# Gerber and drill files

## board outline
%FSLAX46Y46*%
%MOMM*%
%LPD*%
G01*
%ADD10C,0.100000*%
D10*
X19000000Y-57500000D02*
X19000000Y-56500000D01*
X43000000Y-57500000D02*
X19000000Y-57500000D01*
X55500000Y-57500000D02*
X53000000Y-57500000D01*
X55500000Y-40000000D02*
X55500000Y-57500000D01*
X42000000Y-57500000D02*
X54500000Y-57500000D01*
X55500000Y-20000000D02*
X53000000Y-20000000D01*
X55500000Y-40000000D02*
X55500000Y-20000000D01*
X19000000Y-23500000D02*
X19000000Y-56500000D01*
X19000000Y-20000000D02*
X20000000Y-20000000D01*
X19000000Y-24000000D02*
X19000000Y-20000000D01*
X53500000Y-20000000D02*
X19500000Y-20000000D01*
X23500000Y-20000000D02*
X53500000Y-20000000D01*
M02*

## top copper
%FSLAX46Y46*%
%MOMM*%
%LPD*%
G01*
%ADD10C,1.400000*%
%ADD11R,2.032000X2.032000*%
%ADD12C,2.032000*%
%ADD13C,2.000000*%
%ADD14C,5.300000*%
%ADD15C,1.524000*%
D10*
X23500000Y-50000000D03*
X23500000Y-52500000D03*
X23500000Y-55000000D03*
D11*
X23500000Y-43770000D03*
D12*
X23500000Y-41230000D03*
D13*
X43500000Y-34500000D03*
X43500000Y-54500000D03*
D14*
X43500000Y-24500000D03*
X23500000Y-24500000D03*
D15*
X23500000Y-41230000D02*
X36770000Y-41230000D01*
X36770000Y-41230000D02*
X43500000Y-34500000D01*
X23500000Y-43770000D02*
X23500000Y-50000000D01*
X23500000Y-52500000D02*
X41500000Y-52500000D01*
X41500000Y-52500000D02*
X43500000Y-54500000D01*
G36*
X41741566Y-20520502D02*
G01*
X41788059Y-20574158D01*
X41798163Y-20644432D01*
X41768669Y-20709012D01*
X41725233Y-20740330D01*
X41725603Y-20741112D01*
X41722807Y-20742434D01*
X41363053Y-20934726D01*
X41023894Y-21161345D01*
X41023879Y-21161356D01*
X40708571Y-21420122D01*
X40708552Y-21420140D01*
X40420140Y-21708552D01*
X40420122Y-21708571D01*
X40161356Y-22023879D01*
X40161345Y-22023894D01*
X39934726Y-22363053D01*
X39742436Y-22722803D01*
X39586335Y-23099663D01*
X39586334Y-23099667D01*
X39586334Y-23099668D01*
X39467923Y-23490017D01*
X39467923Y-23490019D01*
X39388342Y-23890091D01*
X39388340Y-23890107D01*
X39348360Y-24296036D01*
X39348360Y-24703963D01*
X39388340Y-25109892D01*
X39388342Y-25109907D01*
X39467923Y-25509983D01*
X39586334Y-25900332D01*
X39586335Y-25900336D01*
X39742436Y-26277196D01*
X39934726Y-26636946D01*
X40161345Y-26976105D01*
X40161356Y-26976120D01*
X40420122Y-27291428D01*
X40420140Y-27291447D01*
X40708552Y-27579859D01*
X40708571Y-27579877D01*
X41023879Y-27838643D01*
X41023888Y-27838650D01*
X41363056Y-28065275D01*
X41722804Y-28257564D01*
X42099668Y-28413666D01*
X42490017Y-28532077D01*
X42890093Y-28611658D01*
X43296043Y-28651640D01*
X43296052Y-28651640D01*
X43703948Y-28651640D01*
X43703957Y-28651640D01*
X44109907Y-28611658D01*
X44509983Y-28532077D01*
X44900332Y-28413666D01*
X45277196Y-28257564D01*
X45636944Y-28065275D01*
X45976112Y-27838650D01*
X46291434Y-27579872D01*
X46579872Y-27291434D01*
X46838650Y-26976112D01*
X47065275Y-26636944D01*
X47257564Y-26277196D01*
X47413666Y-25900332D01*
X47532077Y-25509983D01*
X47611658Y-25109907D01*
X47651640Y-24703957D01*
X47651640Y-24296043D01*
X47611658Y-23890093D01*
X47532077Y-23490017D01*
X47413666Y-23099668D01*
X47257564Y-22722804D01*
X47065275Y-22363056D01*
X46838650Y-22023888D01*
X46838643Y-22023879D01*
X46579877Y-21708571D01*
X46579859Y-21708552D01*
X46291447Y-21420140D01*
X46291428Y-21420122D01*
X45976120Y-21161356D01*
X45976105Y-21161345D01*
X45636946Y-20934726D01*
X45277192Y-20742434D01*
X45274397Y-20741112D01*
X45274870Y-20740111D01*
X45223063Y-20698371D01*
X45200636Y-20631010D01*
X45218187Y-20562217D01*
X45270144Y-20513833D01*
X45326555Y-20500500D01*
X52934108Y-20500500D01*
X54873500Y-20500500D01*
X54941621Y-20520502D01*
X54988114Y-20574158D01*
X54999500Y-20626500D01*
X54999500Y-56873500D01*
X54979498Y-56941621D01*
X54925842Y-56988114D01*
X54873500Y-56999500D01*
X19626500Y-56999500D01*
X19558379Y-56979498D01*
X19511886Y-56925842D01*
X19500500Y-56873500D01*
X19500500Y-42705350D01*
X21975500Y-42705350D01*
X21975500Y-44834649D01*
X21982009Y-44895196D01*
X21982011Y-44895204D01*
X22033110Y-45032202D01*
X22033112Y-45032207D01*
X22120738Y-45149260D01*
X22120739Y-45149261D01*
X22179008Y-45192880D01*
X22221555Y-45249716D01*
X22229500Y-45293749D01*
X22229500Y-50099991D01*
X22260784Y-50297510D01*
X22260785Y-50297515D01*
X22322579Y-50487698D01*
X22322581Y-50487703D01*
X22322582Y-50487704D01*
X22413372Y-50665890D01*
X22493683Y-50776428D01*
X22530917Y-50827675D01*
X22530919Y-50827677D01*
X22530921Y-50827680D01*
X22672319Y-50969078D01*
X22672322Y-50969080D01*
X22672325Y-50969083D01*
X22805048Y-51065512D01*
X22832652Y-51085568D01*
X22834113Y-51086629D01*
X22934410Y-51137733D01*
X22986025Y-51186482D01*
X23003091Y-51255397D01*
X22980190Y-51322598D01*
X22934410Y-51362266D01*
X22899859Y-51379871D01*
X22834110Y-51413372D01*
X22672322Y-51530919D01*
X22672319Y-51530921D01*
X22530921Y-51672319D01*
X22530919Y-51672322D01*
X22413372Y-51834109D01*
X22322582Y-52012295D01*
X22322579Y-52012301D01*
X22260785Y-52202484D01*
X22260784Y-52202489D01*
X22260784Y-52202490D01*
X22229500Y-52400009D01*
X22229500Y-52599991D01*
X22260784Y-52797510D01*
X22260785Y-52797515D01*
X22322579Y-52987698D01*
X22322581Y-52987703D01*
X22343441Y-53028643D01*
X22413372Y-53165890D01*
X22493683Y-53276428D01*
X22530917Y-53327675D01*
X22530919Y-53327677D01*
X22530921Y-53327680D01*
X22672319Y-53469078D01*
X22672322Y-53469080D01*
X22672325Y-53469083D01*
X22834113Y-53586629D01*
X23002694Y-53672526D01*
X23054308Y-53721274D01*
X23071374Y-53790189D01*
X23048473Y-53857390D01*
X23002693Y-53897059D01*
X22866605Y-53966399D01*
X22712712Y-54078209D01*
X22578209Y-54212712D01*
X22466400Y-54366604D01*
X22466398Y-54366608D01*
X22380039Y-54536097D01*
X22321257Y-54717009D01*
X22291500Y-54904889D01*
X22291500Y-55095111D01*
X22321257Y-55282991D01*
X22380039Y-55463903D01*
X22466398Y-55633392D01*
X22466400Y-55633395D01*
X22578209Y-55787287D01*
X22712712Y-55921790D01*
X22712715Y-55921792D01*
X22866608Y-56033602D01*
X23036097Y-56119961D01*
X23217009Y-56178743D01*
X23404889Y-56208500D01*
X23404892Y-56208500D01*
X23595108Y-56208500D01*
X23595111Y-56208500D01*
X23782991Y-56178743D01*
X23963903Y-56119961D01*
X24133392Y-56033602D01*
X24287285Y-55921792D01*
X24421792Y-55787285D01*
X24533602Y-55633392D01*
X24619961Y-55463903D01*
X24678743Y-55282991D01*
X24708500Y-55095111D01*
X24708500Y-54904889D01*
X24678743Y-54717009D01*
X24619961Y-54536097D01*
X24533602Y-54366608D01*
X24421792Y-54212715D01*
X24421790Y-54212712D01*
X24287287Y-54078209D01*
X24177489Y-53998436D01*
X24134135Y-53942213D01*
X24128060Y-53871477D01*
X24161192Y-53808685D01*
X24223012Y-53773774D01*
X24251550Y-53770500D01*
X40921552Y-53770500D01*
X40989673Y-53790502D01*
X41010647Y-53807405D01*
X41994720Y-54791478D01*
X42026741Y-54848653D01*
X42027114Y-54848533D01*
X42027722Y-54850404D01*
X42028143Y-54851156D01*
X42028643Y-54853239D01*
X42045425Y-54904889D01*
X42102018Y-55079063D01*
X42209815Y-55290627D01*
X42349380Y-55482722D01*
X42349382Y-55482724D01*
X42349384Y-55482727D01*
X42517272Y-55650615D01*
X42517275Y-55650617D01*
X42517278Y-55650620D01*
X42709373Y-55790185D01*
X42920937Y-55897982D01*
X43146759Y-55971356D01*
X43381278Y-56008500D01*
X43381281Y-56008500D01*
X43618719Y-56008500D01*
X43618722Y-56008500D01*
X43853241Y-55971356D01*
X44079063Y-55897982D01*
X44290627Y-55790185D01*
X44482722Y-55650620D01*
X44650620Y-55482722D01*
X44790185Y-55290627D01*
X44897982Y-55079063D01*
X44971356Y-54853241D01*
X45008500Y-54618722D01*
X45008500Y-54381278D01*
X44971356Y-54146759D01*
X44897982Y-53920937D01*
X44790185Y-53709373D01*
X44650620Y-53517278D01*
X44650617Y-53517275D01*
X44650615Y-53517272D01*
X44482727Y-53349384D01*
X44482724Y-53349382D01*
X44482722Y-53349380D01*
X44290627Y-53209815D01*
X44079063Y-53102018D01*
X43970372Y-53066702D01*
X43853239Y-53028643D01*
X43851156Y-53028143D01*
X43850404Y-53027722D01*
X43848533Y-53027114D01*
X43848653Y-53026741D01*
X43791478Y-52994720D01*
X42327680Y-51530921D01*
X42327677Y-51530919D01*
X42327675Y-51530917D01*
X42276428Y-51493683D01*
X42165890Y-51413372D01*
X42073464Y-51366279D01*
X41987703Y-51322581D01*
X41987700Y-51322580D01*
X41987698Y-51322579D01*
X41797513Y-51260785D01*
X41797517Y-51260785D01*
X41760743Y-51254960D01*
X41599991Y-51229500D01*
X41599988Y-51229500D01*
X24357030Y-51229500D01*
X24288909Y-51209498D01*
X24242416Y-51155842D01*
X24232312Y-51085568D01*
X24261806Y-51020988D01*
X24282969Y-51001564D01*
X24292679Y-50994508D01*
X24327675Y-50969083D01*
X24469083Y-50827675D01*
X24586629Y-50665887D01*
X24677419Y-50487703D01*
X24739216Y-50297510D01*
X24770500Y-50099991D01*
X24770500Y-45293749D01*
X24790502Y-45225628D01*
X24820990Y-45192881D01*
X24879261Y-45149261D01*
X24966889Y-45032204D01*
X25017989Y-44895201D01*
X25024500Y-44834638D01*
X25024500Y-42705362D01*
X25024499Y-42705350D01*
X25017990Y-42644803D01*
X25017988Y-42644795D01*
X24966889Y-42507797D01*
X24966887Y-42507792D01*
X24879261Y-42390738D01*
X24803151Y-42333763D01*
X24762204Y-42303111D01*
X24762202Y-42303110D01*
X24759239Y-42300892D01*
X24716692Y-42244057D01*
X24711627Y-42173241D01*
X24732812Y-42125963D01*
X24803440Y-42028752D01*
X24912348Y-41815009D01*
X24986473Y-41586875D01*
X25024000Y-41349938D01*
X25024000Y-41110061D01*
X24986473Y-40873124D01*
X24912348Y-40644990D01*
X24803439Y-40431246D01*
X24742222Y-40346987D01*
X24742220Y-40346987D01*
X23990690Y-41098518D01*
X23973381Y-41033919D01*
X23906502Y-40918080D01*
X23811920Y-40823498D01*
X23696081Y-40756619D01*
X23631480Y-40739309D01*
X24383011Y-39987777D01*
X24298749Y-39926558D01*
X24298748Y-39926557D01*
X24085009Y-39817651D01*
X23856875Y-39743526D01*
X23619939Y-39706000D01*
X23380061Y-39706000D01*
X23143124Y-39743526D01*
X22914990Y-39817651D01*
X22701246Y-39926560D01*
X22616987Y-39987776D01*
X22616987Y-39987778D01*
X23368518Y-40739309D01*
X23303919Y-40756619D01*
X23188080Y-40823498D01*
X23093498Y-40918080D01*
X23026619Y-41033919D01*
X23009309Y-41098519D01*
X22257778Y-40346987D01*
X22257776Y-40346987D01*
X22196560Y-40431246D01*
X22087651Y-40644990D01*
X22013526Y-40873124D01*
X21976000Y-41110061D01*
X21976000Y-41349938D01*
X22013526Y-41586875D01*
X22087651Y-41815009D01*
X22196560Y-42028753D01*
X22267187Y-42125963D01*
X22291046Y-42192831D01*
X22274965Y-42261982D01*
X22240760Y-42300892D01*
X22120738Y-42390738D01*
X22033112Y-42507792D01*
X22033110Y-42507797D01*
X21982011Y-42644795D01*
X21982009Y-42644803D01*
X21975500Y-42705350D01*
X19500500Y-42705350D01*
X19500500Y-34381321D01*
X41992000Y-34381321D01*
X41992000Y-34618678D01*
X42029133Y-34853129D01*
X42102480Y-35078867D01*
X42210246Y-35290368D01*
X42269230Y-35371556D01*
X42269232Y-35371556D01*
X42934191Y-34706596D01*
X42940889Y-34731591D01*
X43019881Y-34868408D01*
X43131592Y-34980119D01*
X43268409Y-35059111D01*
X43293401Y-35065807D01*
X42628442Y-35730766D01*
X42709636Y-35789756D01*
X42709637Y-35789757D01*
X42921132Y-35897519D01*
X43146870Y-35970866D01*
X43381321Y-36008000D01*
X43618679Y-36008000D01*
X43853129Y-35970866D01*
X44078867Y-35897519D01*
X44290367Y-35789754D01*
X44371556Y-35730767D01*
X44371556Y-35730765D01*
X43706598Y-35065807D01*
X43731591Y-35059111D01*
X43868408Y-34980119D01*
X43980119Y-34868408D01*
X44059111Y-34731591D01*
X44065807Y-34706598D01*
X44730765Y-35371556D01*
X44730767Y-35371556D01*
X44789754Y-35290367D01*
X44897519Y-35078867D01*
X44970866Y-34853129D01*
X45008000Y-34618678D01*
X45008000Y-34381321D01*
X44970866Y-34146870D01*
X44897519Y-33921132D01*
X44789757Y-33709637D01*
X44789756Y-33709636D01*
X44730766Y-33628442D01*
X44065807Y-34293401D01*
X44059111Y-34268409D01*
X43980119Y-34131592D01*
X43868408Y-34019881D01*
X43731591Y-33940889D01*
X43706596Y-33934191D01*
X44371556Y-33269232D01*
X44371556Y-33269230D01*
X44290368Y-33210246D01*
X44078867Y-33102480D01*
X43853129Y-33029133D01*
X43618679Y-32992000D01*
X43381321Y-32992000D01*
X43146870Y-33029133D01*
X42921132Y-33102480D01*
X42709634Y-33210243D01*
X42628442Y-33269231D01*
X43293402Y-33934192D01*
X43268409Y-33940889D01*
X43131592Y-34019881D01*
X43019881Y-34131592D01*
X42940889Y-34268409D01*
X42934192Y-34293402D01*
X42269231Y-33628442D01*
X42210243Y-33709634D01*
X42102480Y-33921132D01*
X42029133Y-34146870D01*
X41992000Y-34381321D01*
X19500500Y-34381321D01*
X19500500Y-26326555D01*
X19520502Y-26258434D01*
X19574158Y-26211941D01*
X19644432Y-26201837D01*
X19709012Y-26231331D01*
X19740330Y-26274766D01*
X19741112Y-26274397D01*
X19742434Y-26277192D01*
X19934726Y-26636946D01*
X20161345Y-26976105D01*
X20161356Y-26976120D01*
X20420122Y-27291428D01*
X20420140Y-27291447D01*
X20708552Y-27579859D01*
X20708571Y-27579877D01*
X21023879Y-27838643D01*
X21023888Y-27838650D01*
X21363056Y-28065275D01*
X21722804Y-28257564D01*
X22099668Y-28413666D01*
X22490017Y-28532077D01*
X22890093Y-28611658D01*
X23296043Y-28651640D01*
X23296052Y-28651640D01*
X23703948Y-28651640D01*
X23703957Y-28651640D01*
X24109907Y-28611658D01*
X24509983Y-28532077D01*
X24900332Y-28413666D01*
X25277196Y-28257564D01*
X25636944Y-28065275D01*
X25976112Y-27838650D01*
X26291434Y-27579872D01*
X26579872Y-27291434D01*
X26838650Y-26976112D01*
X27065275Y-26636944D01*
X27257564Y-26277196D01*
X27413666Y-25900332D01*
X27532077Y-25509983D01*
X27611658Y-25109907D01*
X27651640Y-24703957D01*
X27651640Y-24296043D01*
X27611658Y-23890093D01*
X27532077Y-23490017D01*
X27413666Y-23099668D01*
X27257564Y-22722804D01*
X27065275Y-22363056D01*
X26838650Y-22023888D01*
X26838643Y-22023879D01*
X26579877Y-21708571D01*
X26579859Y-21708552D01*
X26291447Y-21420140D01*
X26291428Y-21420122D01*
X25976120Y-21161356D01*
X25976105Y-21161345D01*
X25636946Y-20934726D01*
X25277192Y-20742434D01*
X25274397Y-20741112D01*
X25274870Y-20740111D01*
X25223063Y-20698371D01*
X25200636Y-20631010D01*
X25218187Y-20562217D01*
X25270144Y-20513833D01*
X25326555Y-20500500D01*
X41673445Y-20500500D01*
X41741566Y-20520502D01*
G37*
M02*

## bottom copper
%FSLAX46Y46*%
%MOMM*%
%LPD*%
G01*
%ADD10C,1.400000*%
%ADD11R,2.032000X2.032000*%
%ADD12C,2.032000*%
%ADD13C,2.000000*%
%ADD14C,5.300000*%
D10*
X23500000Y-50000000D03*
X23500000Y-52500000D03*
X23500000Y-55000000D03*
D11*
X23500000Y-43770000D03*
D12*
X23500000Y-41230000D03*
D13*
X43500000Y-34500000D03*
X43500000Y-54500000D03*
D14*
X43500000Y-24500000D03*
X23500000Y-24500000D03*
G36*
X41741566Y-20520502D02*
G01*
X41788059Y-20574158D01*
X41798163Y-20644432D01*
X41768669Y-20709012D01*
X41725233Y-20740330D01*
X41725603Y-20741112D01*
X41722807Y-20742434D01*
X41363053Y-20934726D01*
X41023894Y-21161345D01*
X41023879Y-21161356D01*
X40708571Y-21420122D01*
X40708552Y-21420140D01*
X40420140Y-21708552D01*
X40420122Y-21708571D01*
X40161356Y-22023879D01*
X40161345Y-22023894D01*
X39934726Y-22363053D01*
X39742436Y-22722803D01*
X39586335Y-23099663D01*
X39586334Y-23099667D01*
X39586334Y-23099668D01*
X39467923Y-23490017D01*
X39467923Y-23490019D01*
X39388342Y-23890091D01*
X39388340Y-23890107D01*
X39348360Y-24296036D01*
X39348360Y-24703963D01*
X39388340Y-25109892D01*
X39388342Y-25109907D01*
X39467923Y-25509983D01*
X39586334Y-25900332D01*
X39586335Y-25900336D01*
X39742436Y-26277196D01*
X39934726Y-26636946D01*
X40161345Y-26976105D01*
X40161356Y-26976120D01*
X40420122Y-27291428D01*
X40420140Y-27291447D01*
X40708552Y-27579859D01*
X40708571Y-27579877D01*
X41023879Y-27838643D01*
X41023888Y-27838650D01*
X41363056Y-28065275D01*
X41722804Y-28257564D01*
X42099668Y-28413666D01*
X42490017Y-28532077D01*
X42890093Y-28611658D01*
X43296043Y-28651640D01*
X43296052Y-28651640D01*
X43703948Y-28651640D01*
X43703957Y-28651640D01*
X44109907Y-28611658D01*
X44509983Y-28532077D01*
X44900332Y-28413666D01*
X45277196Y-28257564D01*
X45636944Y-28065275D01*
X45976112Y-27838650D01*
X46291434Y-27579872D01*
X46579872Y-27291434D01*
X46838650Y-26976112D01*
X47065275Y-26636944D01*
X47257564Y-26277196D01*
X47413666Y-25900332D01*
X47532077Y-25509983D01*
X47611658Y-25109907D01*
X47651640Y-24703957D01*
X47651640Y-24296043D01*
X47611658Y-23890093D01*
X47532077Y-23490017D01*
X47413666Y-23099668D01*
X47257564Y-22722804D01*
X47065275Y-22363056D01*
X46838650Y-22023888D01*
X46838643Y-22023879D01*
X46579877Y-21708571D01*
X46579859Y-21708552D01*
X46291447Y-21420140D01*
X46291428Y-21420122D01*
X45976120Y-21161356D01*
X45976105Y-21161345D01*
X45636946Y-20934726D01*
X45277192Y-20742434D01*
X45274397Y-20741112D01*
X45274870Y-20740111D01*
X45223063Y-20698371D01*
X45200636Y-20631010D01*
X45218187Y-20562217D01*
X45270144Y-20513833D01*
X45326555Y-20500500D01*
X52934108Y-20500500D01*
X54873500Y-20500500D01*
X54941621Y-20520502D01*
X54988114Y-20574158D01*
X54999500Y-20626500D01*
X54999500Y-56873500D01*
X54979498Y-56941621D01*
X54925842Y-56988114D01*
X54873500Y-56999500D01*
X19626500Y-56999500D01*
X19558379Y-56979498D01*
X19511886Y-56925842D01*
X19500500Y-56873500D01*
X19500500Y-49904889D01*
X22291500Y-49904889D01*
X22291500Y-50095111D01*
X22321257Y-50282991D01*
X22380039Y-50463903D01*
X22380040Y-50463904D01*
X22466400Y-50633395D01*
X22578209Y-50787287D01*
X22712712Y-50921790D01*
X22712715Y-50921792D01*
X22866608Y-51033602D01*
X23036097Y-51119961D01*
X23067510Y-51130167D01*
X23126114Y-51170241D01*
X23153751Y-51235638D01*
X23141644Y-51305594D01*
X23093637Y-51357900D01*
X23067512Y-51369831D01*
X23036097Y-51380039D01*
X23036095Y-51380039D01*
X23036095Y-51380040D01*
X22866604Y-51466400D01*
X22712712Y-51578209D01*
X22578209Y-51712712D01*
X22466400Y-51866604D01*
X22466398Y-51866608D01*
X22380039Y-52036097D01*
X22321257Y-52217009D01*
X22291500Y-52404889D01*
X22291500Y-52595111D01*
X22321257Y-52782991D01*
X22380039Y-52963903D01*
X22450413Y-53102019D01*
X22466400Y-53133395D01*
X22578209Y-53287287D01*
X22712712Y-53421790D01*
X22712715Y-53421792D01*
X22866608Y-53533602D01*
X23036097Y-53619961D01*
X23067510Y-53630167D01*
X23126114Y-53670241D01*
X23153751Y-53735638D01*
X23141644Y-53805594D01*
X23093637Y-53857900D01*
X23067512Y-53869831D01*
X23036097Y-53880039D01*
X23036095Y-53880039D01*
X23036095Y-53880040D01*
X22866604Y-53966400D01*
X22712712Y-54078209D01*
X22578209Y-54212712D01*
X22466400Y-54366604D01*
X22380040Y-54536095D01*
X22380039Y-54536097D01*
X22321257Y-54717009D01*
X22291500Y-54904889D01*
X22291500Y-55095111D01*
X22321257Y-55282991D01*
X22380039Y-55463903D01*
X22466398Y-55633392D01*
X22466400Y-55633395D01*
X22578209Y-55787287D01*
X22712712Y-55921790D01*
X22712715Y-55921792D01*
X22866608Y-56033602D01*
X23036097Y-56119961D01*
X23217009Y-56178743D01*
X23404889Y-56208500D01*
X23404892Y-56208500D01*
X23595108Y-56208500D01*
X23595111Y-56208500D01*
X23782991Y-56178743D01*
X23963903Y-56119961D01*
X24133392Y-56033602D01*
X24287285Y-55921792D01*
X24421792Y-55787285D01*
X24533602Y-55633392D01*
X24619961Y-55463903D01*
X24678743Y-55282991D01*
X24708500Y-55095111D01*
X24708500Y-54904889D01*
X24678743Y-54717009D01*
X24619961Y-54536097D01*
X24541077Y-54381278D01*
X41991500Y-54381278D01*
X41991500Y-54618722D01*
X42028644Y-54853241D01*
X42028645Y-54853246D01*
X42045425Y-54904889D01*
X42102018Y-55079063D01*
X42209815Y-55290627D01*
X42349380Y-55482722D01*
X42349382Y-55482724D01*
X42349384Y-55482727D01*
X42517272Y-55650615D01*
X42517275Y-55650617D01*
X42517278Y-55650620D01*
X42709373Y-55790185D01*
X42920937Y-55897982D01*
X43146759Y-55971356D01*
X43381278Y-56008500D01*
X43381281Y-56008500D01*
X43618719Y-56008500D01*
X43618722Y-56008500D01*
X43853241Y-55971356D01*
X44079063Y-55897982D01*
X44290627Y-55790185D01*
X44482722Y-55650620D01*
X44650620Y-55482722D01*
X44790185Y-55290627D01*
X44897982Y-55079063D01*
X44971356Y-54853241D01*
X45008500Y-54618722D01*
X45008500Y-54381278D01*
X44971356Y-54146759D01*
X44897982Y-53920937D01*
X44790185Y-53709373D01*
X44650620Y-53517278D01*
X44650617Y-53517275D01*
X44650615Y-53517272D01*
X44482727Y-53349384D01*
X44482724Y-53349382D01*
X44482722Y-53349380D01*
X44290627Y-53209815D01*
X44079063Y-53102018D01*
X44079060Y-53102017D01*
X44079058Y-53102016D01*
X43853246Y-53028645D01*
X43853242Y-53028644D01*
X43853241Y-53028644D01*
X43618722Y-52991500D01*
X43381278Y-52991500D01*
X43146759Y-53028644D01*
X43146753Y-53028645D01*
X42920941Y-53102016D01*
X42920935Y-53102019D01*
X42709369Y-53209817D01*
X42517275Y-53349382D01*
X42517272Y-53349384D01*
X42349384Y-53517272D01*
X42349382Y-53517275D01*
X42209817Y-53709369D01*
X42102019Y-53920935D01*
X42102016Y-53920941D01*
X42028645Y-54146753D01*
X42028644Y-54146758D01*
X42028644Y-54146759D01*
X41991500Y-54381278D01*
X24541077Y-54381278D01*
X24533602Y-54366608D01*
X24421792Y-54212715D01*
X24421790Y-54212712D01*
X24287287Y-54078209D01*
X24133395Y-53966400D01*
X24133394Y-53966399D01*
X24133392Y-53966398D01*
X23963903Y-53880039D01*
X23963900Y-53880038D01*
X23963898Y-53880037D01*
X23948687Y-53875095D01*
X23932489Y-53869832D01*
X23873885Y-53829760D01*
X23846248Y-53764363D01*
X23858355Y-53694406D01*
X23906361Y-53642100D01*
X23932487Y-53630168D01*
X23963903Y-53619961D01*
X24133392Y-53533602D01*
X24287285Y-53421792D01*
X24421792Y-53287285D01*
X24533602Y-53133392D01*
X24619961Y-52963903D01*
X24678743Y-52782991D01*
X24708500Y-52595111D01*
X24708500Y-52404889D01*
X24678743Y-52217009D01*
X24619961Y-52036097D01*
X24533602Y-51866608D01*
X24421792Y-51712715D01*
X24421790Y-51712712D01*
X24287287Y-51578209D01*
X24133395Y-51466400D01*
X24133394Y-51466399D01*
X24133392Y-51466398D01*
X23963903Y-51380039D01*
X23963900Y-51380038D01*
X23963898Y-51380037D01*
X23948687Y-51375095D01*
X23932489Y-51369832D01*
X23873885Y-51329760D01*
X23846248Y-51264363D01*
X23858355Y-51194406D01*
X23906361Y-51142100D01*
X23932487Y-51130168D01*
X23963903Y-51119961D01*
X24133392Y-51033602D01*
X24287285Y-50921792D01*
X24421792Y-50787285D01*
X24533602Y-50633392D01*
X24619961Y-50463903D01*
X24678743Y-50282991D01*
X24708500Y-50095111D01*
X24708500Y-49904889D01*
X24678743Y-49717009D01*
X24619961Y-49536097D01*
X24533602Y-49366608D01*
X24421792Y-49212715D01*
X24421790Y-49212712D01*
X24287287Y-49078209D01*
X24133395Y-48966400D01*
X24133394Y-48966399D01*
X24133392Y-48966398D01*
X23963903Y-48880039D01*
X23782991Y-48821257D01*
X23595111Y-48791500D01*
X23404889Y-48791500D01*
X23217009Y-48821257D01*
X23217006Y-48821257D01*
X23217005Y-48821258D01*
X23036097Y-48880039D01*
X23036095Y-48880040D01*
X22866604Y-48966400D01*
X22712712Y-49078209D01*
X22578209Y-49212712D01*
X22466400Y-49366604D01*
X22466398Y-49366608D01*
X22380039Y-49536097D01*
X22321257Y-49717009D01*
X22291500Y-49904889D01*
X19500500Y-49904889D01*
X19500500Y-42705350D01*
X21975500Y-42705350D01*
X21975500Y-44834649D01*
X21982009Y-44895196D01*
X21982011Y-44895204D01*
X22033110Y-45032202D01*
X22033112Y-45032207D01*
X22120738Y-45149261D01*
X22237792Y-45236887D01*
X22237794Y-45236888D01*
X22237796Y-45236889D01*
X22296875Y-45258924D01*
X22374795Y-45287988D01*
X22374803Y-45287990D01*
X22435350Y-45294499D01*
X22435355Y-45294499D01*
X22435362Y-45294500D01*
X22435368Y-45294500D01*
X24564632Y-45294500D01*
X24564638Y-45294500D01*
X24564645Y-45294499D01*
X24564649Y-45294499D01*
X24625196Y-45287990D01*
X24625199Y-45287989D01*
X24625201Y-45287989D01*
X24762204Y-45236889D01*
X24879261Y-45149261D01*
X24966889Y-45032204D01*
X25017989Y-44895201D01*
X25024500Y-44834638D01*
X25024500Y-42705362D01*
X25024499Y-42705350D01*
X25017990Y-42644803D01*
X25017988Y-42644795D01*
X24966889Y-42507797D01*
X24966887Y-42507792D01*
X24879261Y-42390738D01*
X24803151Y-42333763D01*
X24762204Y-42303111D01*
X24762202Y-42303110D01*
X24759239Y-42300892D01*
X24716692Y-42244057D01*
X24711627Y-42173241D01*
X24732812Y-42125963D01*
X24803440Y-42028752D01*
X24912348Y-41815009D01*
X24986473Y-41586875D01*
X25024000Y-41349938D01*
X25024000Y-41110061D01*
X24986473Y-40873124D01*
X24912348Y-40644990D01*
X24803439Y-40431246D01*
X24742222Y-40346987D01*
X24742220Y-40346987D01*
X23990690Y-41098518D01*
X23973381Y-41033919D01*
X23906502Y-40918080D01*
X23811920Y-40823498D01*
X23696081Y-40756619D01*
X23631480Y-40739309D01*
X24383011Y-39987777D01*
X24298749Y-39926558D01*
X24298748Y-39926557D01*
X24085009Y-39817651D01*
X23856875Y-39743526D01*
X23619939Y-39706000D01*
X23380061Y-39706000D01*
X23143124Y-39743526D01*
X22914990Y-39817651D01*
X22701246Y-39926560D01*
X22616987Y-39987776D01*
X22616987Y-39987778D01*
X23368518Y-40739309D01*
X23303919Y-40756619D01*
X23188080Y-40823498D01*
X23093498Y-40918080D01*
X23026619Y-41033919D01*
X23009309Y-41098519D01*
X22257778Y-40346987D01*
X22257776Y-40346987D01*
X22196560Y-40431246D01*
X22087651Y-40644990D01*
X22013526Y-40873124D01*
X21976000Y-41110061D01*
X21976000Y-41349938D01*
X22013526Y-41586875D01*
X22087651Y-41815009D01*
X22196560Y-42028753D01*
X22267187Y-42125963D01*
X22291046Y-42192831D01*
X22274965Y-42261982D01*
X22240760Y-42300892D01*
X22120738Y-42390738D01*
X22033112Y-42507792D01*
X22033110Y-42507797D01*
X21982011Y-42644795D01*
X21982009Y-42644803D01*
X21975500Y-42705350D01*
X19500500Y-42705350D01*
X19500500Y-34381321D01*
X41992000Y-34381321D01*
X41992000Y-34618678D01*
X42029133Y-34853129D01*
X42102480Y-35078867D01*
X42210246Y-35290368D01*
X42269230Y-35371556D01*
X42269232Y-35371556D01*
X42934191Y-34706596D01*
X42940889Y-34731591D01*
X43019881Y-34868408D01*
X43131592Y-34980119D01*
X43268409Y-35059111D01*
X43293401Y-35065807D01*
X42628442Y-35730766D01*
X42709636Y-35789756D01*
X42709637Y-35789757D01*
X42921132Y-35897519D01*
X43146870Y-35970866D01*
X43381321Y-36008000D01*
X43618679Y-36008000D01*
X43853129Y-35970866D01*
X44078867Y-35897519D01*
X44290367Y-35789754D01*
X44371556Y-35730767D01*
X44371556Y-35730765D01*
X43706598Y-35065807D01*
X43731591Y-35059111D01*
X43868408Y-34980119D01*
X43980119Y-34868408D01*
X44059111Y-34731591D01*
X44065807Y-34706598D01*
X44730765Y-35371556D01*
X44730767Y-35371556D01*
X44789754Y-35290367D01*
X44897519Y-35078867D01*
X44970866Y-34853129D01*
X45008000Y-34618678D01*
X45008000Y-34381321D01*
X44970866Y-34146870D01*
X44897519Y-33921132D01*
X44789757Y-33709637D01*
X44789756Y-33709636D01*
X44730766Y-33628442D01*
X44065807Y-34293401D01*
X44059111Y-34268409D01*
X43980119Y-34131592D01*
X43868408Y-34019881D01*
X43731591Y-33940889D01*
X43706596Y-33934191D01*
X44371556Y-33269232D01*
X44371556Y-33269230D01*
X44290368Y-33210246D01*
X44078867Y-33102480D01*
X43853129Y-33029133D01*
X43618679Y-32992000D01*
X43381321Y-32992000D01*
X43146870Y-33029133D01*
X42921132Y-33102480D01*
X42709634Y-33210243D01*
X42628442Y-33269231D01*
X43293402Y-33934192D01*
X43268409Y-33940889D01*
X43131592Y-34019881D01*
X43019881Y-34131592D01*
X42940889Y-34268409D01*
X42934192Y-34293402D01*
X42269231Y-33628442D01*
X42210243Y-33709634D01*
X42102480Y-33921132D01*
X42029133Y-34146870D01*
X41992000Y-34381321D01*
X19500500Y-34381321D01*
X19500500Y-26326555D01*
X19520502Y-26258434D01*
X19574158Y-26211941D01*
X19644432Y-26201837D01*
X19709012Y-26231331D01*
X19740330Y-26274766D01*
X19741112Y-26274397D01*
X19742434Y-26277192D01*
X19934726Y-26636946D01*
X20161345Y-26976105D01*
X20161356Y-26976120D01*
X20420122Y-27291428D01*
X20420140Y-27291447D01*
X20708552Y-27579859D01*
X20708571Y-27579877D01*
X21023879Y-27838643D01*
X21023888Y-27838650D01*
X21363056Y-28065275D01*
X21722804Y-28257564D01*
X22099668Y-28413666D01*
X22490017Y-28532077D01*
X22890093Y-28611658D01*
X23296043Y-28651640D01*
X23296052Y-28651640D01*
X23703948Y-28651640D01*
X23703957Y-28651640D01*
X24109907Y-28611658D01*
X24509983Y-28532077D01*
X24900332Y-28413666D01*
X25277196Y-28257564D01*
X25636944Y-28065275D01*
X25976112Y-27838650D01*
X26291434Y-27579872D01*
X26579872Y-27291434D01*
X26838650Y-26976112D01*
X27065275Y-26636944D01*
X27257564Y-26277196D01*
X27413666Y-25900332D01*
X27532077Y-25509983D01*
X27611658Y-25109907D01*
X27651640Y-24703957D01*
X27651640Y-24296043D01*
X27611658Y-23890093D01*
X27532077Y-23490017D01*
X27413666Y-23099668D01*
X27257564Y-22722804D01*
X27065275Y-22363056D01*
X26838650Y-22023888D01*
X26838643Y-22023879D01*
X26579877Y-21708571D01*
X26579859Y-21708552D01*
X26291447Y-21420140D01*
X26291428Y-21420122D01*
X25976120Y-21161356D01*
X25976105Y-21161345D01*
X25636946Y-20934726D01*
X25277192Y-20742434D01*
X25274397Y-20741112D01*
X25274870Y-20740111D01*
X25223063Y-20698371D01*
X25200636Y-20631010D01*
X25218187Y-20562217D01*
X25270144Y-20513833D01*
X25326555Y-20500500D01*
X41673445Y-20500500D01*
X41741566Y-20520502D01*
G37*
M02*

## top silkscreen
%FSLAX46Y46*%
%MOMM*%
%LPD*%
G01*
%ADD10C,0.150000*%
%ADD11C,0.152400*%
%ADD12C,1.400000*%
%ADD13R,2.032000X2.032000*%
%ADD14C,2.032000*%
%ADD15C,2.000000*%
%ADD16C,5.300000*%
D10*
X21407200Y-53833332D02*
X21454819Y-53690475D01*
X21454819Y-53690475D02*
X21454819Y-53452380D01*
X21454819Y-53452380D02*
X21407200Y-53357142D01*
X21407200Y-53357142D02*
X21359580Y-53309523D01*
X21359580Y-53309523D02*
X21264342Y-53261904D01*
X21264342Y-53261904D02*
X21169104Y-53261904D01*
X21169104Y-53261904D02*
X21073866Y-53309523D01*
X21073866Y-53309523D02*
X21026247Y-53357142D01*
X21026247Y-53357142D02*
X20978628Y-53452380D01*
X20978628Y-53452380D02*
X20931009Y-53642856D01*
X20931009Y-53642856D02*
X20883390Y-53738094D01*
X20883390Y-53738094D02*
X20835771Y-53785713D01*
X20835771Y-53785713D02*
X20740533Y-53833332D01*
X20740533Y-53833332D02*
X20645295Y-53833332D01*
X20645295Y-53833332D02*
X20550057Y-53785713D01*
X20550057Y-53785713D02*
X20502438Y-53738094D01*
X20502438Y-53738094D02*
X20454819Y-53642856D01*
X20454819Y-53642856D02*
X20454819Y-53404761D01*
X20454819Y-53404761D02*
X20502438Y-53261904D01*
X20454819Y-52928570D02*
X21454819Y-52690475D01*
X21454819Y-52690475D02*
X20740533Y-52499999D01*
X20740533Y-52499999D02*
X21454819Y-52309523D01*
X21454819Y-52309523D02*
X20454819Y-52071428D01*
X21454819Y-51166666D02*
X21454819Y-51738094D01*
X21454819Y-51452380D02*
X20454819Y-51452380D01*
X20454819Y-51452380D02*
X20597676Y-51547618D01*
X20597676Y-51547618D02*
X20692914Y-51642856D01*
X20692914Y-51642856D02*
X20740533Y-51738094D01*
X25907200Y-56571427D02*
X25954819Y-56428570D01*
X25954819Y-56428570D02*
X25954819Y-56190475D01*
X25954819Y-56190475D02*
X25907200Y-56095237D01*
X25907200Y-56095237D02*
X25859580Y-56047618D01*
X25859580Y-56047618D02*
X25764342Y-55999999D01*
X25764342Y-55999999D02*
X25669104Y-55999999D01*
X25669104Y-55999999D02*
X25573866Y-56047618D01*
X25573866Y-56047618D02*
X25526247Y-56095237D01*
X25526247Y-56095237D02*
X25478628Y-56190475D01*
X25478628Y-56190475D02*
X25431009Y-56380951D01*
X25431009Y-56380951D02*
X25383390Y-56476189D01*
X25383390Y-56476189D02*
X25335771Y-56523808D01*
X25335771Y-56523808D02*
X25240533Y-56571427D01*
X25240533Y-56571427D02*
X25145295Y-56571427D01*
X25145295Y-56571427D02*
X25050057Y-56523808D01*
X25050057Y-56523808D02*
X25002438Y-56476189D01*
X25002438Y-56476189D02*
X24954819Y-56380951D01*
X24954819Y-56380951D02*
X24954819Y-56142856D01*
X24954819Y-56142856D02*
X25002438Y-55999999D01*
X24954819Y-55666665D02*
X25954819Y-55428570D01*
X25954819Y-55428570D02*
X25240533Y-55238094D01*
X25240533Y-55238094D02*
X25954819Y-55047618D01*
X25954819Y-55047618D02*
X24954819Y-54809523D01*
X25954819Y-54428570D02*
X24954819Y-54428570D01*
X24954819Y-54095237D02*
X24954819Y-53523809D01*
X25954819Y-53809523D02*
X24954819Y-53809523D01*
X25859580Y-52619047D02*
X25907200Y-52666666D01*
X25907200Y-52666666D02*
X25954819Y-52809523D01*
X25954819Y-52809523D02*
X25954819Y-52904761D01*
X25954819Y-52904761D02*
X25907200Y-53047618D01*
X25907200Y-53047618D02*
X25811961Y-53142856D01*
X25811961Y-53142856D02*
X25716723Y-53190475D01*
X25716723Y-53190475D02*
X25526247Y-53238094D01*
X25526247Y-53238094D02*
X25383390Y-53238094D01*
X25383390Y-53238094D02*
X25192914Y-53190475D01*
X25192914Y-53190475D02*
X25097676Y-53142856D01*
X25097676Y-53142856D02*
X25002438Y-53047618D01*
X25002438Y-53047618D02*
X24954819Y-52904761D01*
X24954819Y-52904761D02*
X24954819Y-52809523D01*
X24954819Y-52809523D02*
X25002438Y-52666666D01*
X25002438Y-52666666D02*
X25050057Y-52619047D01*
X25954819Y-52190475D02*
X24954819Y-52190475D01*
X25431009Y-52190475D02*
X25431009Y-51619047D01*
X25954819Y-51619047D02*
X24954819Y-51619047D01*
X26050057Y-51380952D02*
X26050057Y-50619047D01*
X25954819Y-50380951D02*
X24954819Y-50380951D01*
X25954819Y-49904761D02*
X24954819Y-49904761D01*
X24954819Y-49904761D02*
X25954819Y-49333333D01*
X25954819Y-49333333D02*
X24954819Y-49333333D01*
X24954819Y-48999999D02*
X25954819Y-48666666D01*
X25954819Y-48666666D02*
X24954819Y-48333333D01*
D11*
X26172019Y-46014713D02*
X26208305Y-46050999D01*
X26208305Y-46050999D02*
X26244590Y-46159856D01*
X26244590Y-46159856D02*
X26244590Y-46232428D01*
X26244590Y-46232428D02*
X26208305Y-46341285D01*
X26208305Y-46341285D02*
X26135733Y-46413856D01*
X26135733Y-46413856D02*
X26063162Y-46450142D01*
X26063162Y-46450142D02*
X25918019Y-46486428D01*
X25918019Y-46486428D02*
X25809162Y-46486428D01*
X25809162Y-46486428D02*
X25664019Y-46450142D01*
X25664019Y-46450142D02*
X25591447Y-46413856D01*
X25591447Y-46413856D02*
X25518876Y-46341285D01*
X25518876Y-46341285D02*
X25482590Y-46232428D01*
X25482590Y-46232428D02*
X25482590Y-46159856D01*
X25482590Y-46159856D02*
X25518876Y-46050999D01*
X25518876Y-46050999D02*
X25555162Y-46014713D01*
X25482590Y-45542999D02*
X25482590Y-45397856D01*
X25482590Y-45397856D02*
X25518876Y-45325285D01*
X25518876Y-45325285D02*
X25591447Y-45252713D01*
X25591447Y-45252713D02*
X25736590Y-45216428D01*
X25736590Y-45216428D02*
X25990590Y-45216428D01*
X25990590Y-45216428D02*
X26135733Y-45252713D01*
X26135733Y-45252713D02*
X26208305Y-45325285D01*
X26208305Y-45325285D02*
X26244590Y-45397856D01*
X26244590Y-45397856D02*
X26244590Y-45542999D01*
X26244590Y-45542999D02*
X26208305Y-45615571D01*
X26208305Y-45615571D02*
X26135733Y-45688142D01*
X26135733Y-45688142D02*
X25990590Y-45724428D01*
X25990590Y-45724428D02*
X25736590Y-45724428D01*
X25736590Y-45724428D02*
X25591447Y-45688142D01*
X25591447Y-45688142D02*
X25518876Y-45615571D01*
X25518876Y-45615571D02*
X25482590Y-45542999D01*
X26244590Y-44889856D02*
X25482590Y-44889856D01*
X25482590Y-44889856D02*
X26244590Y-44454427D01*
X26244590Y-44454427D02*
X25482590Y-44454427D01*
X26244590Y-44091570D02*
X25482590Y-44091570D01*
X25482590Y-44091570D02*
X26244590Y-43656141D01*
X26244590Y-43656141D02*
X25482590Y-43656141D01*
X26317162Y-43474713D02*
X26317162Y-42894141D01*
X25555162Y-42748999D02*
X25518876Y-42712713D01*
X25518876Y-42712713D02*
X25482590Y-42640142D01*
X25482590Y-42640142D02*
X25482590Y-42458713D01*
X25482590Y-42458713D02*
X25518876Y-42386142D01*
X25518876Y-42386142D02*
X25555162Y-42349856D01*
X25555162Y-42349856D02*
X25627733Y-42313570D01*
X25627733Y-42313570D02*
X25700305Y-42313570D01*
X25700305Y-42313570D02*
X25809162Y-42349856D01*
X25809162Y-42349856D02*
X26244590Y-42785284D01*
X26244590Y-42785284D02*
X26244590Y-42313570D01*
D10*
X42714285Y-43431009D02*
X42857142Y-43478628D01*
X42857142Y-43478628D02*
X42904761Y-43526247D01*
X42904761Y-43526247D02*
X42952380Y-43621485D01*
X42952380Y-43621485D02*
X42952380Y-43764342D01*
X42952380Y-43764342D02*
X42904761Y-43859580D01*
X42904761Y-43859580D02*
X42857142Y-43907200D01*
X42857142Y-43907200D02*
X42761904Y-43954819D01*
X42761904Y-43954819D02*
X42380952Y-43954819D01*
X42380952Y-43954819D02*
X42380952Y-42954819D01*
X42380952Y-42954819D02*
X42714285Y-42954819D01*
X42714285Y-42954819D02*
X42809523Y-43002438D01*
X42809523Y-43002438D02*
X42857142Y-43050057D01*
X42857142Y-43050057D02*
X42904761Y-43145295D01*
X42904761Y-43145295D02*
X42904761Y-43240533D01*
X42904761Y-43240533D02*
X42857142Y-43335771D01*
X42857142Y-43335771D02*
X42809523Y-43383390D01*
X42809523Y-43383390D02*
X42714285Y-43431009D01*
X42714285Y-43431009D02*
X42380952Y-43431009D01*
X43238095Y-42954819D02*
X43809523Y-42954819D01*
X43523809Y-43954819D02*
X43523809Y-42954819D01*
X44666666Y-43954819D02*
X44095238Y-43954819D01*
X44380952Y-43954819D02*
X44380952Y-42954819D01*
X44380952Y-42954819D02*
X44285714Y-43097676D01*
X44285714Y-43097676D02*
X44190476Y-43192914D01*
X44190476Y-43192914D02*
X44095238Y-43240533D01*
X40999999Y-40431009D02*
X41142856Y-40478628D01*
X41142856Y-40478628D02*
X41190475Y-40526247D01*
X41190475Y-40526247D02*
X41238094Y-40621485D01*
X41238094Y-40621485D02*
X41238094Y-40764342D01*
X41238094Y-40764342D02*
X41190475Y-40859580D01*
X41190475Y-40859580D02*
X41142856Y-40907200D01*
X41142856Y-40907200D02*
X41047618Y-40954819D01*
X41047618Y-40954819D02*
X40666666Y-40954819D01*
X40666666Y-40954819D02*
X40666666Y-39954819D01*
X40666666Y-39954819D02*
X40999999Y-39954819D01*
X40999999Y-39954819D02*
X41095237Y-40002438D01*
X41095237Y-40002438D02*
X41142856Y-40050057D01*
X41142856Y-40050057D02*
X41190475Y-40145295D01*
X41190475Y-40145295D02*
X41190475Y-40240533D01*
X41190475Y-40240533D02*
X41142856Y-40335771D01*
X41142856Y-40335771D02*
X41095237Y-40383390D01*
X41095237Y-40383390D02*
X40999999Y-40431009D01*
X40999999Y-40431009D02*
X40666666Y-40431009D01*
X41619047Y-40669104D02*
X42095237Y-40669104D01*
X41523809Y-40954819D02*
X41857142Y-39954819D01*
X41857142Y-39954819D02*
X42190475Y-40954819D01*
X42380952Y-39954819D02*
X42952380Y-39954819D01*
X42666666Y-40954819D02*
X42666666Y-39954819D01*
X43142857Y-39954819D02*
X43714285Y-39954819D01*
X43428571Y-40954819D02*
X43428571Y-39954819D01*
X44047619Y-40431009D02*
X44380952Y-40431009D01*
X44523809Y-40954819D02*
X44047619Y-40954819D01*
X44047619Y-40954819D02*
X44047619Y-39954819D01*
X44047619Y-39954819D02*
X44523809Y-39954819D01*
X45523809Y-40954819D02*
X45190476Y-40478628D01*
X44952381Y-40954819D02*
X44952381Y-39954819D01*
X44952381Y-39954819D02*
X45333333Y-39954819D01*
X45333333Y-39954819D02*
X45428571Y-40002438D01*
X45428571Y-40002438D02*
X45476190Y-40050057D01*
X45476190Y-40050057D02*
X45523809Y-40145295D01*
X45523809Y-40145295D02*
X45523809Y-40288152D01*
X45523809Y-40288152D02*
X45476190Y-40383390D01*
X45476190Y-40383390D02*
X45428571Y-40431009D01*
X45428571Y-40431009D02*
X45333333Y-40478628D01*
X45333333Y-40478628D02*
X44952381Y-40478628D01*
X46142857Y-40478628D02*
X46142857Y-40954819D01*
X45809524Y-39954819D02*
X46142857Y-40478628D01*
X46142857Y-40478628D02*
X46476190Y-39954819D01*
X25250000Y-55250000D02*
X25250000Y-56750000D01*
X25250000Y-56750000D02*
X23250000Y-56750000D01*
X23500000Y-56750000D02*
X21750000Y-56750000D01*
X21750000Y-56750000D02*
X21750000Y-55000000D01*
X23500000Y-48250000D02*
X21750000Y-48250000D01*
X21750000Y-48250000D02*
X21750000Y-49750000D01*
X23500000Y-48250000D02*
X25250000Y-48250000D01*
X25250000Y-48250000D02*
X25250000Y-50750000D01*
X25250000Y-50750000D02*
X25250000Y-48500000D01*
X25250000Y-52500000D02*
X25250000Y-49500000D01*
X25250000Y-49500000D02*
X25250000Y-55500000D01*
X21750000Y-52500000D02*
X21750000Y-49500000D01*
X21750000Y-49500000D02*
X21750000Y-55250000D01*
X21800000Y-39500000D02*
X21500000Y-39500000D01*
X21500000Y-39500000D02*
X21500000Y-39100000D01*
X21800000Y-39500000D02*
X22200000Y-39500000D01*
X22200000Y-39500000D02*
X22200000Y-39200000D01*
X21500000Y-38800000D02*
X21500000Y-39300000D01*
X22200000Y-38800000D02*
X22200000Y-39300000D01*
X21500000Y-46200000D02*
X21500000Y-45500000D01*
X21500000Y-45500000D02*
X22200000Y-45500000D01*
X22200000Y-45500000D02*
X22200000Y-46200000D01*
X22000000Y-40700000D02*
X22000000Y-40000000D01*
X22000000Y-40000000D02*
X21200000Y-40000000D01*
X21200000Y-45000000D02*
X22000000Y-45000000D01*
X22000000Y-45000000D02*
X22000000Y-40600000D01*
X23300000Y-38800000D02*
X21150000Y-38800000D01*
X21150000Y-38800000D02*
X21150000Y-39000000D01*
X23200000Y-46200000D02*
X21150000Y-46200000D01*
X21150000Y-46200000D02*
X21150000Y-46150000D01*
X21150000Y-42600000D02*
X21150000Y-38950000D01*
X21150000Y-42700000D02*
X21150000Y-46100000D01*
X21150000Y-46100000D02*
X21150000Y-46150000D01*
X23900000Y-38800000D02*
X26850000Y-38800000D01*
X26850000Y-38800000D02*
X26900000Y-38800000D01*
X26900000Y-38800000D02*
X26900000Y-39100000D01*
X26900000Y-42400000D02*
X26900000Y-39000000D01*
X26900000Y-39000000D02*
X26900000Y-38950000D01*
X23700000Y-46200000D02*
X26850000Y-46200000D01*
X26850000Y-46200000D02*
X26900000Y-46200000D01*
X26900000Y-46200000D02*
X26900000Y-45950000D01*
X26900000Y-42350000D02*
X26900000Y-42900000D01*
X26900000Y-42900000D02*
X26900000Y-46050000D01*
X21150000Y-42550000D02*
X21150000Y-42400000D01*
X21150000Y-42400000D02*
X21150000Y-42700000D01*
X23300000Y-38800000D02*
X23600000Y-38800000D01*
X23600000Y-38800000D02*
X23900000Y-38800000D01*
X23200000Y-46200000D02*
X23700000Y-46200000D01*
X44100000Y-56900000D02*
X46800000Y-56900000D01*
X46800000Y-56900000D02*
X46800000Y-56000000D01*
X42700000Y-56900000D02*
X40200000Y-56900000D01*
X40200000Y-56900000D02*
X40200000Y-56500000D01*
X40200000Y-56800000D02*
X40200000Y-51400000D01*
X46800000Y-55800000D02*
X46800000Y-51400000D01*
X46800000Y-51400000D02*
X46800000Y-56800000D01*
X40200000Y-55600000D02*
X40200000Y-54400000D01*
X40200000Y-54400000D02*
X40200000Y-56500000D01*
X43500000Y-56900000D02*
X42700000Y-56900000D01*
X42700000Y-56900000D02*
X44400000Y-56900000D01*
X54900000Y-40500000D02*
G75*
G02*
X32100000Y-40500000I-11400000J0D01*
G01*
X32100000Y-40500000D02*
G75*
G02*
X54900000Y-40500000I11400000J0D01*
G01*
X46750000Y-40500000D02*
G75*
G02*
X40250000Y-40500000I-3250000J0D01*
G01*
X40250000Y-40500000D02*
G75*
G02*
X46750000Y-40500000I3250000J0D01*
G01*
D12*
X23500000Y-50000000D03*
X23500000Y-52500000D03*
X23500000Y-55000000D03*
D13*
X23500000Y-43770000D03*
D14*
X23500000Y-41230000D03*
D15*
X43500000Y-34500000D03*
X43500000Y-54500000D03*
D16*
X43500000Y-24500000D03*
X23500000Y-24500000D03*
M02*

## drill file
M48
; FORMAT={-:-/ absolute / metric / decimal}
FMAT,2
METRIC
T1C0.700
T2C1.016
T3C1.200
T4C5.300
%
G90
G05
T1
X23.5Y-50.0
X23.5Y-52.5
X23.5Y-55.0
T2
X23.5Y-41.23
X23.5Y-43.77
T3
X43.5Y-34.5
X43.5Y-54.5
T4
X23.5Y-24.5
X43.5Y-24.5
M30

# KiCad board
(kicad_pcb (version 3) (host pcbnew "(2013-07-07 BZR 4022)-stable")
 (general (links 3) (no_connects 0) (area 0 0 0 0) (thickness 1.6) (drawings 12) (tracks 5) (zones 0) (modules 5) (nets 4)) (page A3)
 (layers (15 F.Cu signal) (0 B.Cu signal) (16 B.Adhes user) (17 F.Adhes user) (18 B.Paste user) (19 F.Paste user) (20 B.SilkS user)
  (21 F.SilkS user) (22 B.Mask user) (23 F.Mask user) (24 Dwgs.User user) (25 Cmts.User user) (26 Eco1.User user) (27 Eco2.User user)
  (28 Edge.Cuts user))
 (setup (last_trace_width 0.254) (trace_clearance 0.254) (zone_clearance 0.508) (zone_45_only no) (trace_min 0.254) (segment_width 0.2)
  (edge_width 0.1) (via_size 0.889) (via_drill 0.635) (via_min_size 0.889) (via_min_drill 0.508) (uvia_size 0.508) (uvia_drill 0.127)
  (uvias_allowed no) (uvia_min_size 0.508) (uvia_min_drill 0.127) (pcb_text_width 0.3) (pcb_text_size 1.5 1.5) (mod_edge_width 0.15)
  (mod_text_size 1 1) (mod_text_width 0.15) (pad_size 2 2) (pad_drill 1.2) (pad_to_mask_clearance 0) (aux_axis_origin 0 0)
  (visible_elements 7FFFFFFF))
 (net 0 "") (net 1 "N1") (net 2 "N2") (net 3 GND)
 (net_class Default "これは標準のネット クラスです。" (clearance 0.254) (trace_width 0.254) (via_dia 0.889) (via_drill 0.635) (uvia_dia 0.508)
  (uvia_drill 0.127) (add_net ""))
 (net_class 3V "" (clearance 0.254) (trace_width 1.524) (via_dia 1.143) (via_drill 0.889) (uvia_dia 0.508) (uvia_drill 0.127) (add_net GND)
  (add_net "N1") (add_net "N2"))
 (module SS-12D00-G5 (layer F.Cu) (at 23.5 52.5 270)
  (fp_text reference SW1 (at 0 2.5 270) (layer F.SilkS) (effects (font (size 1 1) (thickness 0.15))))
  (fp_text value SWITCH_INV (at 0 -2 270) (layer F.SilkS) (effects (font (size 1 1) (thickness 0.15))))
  (fp_line (start 2.75 -1.75) (end 4.25 -1.75) (layer F.SilkS) (width 0.15))
  (fp_line (start 4.25 -1.75) (end 4.25 0.25) (layer F.SilkS) (width 0.15))
  (fp_line (start 4.25 0) (end 4.25 1.75) (layer F.SilkS) (width 0.15))
  (fp_line (start 4.25 1.75) (end 2.5 1.75) (layer F.SilkS) (width 0.15))
  (fp_line (start -4.25 0) (end -4.25 1.75) (layer F.SilkS) (width 0.15))
  (fp_line (start -4.25 1.75) (end -2.75 1.75) (layer F.SilkS) (width 0.15))
  (fp_line (start -4.25 0) (end -4.25 -1.75) (layer F.SilkS) (width 0.15))
  (fp_line (start -4.25 -1.75) (end -1.75 -1.75) (layer F.SilkS) (width 0.15))
  (fp_line (start -1.75 -1.75) (end -4 -1.75) (layer F.SilkS) (width 0.15))
  (fp_line (start 0 -1.75) (end -3 -1.75) (layer F.SilkS) (width 0.15))
  (fp_line (start -3 -1.75) (end 3 -1.75) (layer F.SilkS) (width 0.15))
  (fp_line (start 0 1.75) (end -3 1.75) (layer F.SilkS) (width 0.15))
  (fp_line (start -3 1.75) (end 2.75 1.75) (layer F.SilkS) (width 0.15))
  (pad 1 thru_hole circle (at -2.5 0 270) (size 1.4 1.4) (drill 0.7) (layers *.Cu *.Mask F.SilkS) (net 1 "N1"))
  (pad 2 thru_hole circle (at 0 0 270) (size 1.4 1.4) (drill 0.7) (layers *.Cu *.Mask F.SilkS) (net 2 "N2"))
  (pad 3 thru_hole circle (at 2.5 0 270) (size 1.4 1.4) (drill 0.7) (layers *.Cu *.Mask F.SilkS)))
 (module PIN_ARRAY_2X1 (layer F.Cu) (at 23.5 42.5 90)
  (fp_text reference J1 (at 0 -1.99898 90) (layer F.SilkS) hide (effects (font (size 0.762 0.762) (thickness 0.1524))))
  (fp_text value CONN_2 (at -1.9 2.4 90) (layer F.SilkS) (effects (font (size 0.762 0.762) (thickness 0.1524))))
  (fp_line (start 3 -1.7) (end 3 -2) (layer F.SilkS) (width 0.15))
  (fp_line (start 3 -2) (end 3.4 -2) (layer F.SilkS) (width 0.15))
  (fp_line (start 3 -1.7) (end 3 -1.3) (layer F.SilkS) (width 0.15))
  (fp_line (start 3 -1.3) (end 3.3 -1.3) (layer F.SilkS) (width 0.15))
  (fp_line (start 3.7 -2) (end 3.2 -2) (layer F.SilkS) (width 0.15))
  (fp_line (start 3.7 -1.3) (end 3.2 -1.3) (layer F.SilkS) (width 0.15))
  (fp_line (start -3.7 -2) (end -3 -2) (layer F.SilkS) (width 0.15))
  (fp_line (start -3 -2) (end -3 -1.3) (layer F.SilkS) (width 0.15))
  (fp_line (start -3 -1.3) (end -3.7 -1.3) (layer F.SilkS) (width 0.15))
  (fp_line (start 1.8 -1.5) (end 2.5 -1.5) (layer F.SilkS) (width 0.15))
  (fp_line (start 2.5 -1.5) (end 2.5 -2.3) (layer F.SilkS) (width 0.15))
  (fp_line (start -2.5 -2.3) (end -2.5 -1.5) (layer F.SilkS) (width 0.15))
  (fp_line (start -2.5 -1.5) (end 1.9 -1.5) (layer F.SilkS) (width 0.15))
  (fp_line (start 3.7 -0.2) (end 3.7 -2.35) (layer F.SilkS) (width 0.15))
  (fp_line (start 3.7 -2.35) (end 3.5 -2.35) (layer F.SilkS) (width 0.15))
  (fp_line (start -3.7 -0.3) (end -3.7 -2.35) (layer F.SilkS) (width 0.15))
  (fp_line (start -3.7 -2.35) (end -3.65 -2.35) (layer F.SilkS) (width 0.15))
  (fp_line (start -0.1 -2.35) (end 3.55 -2.35) (layer F.SilkS) (width 0.15))
  (fp_line (start -0.2 -2.35) (end -3.6 -2.35) (layer F.SilkS) (width 0.15))
  (fp_line (start -3.6 -2.35) (end -3.65 -2.35) (layer F.SilkS) (width 0.15))
  (fp_line (start 3.7 0.4) (end 3.7 3.35) (layer F.SilkS) (width 0.15))
  (fp_line (start 3.7 3.35) (end 3.7 3.4) (layer F.SilkS) (width 0.15))
  (fp_line (start 3.7 3.4) (end 3.4 3.4) (layer F.SilkS) (width 0.15))
  (fp_line (start 0.1 3.4) (end 3.5 3.4) (layer F.SilkS) (width 0.15))
  (fp_line (start 3.5 3.4) (end 3.55 3.4) (layer F.SilkS) (width 0.15))
  (fp_line (start -3.7 0.2) (end -3.7 3.35) (layer F.SilkS) (width 0.15))
  (fp_line (start -3.7 3.35) (end -3.7 3.4) (layer F.SilkS) (width 0.15))
  (fp_line (start -3.7 3.4) (end -3.45 3.4) (layer F.SilkS) (width 0.15))
  (fp_line (start 0.15 3.4) (end -0.4 3.4) (layer F.SilkS) (width 0.15))
  (fp_line (start -0.4 3.4) (end -3.55 3.4) (layer F.SilkS) (width 0.15))
  (fp_line (start -0.05 -2.35) (end 0.1 -2.35) (layer F.SilkS) (width 0.15))
  (fp_line (start 0.1 -2.35) (end -0.2 -2.35) (layer F.SilkS) (width 0.15))
  (fp_line (start 3.7 -0.2) (end 3.7 0.1) (layer F.SilkS) (width 0.15))
  (fp_line (start 3.7 0.1) (end 3.7 0.4) (layer F.SilkS) (width 0.15))
  (fp_line (start -3.7 -0.3) (end -3.7 0.2) (layer F.SilkS) (width 0.15))
  (pad 1 thru_hole rect (at -1.27 0 90) (size 2.032 2.032) (drill 1.016) (layers *.Cu *.Mask F.SilkS) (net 1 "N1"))
  (pad 2 thru_hole circle (at 1.27 0 90) (size 2.032 2.032) (drill 1.016) (layers *.Cu *.Mask F.SilkS) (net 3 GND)))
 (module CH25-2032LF (layer F.Cu) (at 43.5 40.5)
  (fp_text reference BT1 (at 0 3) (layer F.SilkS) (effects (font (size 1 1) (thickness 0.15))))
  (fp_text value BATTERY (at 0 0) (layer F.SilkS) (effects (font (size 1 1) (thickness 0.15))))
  (fp_line (start 0.6 16.4) (end 3.3 16.4) (layer F.SilkS) (width 0.15))
  (fp_line (start 3.3 16.4) (end 3.3 15.5) (layer F.SilkS) (width 0.15))
  (fp_line (start -0.8 16.4) (end -3.3 16.4) (layer F.SilkS) (width 0.15))
  (fp_line (start -3.3 16.4) (end -3.3 16) (layer F.SilkS) (width 0.15))
  (fp_line (start -3.3 16.3) (end -3.3 10.9) (layer F.SilkS) (width 0.15))
  (fp_line (start 3.3 15.3) (end 3.3 10.9) (layer F.SilkS) (width 0.15))
  (fp_line (start 3.3 10.9) (end 3.3 16.3) (layer F.SilkS) (width 0.15))
  (fp_line (start -3.3 15.1) (end -3.3 13.9) (layer F.SilkS) (width 0.15))
  (fp_line (start -3.3 13.9) (end -3.3 16) (layer F.SilkS) (width 0.15))
  (fp_line (start 0 16.4) (end -0.8 16.4) (layer F.SilkS) (width 0.15))
  (fp_line (start -0.8 16.4) (end 0.9 16.4) (layer F.SilkS) (width 0.15))
  (fp_circle (center 0 0) (end 11.4 0) (layer F.SilkS) (width 0.15))
  (fp_circle (center 0 0) (end 3.25 0) (layer F.SilkS) (width 0.15))
  (pad 2 thru_hole circle (at 0 -6) (size 2 2) (drill 1.2) (layers *.Cu *.Mask F.SilkS) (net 3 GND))
  (pad 1 thru_hole circle (at 0 14) (size 2 2) (drill 1.2) (layers *.Cu *.Mask F.SilkS) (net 2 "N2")))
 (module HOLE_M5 (layer F.Cu) (at 43.5 24.5)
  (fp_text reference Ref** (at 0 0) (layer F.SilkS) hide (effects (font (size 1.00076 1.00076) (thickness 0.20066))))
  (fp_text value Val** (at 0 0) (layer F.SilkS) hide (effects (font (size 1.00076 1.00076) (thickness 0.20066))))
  (pad "" thru_hole circle (at 0 0) (size 5.3 5.3) (drill 5.3) (layers *.Cu *.Mask F.SilkS) (clearance 1.50114)))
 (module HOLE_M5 (layer F.Cu) (at 23.5 24.5)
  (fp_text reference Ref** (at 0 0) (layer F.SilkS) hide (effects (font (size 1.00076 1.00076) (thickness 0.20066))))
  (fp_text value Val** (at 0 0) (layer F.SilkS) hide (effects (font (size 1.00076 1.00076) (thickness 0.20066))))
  (pad "" thru_hole circle (at 0 0) (size 5.3 5.3) (drill 5.3) (layers *.Cu *.Mask F.SilkS) (clearance 1.50114)))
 (gr_line (start 19 57.5) (end 19 56.5) (angle 90) (layer Edge.Cuts) (width 0.1))
 (gr_line (start 43 57.5) (end 19 57.5) (angle 90) (layer Edge.Cuts) (width 0.1))
 (gr_line (start 55.5 57.5) (end 53 57.5) (angle 90) (layer Edge.Cuts) (width 0.1))
 (gr_line (start 55.5 40) (end 55.5 57.5) (angle 90) (layer Edge.Cuts) (width 0.1))
 (gr_line (start 42 57.5) (end 54.5 57.5) (angle 90) (layer Edge.Cuts) (width 0.1))
 (gr_line (start 55.5 20) (end 53 20) (angle 90) (layer Edge.Cuts) (width 0.1))
 (gr_line (start 55.5 40) (end 55.5 20) (angle 90) (layer Edge.Cuts) (width 0.1))
 (gr_line (start 19 23.5) (end 19 56.5) (angle 90) (layer Edge.Cuts) (width 0.1))
 (gr_line (start 19 20) (end 20 20) (angle 90) (layer Edge.Cuts) (width 0.1))
 (gr_line (start 19 24) (end 19 20) (angle 90) (layer Edge.Cuts) (width 0.1))
 (gr_line (start 53.5 20) (end 19.5 20) (angle 90) (layer Edge.Cuts) (width 0.1))
 (gr_line (start 23.5 20) (end 53.5 20) (angle 90) (layer Edge.Cuts) (width 0.1))
 (segment (start 23.5 41.23) (end 36.77 41.23) (width 1.524) (layer F.Cu) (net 3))
 (segment (start 36.77 41.23) (end 43.5 34.5) (width 1.524) (layer F.Cu) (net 3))
 (segment (start 23.5 43.77) (end 23.5 50) (width 1.524) (layer F.Cu) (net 1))
 (segment (start 23.5 52.5) (end 41.5 52.5) (width 1.524) (layer F.Cu) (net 2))
 (segment (start 41.5 52.5) (end 43.5 54.5) (width 1.524) (layer F.Cu) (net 2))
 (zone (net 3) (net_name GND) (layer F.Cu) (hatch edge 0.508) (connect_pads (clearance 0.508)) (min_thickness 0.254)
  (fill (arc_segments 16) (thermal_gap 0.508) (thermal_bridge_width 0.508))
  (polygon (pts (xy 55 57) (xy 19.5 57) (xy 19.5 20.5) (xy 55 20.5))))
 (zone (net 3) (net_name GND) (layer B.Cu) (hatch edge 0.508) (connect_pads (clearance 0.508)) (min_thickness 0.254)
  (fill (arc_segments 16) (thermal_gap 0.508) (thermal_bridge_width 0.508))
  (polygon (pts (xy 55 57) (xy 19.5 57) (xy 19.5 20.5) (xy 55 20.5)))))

